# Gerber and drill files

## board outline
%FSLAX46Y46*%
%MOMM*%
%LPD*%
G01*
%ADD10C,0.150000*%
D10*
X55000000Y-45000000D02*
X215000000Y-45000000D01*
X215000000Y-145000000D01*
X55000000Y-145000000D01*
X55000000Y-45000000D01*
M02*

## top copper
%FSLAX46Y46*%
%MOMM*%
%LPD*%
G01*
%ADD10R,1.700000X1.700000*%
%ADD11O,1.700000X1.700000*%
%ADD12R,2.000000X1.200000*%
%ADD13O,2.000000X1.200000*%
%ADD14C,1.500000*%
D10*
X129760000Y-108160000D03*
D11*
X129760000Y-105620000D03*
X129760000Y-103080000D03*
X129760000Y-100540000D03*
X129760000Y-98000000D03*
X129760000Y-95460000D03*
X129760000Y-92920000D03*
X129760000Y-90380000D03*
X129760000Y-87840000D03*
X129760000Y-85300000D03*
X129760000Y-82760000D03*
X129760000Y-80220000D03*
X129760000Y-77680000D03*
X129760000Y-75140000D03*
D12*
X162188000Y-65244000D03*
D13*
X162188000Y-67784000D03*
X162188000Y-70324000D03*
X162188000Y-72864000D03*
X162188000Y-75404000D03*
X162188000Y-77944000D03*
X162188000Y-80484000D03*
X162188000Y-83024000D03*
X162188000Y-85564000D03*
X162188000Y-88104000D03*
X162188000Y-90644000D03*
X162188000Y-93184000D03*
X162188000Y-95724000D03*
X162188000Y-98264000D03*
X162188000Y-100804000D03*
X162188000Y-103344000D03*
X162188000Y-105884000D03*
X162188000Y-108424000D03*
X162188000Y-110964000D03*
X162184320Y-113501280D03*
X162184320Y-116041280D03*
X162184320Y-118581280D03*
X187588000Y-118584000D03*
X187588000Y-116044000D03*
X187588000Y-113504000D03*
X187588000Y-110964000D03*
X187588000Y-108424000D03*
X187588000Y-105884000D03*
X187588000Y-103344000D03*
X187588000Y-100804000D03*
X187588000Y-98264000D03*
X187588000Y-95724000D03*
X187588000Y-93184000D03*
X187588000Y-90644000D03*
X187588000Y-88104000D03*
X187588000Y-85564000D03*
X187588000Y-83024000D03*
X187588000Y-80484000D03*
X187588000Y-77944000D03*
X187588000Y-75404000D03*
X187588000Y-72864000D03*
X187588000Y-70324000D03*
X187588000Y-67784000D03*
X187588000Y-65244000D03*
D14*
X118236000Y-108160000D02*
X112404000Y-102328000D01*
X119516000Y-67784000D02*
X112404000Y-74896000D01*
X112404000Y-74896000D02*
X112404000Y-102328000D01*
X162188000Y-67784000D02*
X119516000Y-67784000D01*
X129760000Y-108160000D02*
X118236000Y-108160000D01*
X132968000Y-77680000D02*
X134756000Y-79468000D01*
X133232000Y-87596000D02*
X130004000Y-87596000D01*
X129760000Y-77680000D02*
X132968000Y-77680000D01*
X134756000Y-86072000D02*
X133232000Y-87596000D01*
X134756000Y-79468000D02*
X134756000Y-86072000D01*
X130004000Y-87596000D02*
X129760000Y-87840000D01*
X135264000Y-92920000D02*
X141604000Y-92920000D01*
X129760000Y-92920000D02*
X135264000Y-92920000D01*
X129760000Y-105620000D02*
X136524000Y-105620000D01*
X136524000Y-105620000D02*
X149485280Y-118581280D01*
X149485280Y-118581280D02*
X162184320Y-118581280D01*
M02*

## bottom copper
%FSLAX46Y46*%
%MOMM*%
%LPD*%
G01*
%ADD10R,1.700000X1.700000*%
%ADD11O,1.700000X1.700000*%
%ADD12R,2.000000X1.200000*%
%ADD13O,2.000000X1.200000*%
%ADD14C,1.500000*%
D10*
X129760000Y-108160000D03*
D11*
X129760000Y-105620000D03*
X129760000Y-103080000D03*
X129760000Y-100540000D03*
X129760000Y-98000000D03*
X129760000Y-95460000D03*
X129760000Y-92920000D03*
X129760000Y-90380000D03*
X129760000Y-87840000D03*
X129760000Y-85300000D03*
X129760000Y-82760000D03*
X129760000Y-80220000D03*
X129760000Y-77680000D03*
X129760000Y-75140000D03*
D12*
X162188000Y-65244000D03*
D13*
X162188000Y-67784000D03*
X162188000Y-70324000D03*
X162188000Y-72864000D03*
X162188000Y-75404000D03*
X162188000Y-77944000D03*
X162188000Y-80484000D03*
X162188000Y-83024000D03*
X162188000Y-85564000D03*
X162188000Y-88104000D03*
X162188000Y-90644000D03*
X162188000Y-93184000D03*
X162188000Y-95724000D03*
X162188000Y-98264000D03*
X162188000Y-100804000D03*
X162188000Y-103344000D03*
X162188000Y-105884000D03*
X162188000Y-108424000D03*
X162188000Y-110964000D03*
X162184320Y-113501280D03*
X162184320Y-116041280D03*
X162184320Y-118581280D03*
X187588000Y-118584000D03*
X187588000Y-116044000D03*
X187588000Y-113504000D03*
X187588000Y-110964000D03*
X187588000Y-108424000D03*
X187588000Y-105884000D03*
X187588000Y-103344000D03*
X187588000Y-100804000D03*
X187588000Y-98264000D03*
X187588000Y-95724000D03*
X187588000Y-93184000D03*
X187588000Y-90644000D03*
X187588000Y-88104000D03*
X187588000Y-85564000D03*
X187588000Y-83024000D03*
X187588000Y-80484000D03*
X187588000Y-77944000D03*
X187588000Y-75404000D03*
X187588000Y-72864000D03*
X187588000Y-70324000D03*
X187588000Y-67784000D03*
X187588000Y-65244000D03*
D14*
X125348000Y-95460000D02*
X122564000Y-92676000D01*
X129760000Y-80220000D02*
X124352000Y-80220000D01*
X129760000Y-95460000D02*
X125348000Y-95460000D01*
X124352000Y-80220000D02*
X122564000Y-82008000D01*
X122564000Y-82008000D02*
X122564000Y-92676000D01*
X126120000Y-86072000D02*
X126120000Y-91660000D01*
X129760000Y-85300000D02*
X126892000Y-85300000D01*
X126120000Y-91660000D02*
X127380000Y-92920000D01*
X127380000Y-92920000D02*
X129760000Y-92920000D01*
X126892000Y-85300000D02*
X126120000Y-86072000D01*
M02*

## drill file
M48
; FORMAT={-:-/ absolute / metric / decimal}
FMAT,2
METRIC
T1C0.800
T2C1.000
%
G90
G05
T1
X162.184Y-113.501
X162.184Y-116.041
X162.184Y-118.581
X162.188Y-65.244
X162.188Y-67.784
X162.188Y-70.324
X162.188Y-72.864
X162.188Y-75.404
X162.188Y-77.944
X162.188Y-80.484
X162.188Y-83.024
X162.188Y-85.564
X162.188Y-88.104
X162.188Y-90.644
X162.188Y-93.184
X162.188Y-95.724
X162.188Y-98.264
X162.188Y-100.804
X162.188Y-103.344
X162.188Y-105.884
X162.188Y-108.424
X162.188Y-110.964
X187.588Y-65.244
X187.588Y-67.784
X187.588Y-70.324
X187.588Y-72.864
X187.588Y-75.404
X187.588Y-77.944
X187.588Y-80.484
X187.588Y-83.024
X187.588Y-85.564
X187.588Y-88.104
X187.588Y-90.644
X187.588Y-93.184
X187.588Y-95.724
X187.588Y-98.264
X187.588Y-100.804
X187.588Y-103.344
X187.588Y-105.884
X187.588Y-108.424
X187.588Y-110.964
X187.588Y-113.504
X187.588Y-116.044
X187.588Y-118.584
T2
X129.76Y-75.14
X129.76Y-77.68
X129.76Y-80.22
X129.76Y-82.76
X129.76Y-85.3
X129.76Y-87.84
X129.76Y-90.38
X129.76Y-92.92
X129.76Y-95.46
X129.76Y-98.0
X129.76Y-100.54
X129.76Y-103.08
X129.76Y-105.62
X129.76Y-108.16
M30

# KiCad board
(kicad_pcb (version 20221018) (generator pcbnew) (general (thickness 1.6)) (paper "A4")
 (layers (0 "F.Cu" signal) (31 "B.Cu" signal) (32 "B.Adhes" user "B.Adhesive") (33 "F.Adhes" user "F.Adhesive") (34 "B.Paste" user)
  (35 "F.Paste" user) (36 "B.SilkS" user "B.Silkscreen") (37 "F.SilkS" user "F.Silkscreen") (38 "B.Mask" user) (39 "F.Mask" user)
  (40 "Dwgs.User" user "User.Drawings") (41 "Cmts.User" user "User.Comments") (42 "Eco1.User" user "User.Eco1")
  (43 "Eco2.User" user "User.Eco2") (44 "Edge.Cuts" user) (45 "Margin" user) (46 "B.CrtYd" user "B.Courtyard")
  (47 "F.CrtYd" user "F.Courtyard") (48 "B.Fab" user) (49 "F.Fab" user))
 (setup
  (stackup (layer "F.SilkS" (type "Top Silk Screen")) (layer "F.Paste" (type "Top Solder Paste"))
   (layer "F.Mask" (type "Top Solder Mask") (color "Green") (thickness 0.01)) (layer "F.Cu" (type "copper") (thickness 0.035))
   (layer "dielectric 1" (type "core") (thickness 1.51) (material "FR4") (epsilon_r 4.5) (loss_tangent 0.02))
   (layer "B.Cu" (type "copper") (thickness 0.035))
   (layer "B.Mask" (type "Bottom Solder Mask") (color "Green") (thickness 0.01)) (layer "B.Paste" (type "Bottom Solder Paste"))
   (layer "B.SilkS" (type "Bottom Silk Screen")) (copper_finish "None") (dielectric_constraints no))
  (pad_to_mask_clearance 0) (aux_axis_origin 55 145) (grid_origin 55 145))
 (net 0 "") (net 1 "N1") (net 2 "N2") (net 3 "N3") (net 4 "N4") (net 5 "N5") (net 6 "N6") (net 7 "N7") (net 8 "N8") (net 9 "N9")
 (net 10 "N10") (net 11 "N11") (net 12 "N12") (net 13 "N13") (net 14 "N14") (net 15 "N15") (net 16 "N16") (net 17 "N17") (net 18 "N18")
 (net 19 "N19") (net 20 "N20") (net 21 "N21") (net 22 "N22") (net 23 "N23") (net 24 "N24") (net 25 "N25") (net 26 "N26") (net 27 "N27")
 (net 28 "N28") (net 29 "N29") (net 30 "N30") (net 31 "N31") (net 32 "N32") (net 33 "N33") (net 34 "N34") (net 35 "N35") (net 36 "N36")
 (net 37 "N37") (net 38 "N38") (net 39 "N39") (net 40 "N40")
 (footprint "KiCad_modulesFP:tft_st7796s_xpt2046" (layer "F.Cu") (at 129.76 108.16 180)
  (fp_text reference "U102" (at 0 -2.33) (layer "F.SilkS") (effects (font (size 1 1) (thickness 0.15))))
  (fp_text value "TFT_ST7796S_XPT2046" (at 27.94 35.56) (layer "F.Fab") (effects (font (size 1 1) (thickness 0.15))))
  (pad "1" thru_hole rect (at 0 0 180) (size 1.7 1.7) (drill 1) (layers "*.Cu" "*.Mask") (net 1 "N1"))
  (pad "2" thru_hole oval (at 0 2.54 180) (size 1.7 1.7) (drill 1) (layers "*.Cu" "*.Mask") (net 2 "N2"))
  (pad "3" thru_hole oval (at 0 5.08 180) (size 1.7 1.7) (drill 1) (layers "*.Cu" "*.Mask") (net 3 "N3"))
  (pad "4" thru_hole oval (at 0 7.62 180) (size 1.7 1.7) (drill 1) (layers "*.Cu" "*.Mask") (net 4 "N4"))
  (pad "5" thru_hole oval (at 0 10.16 180) (size 1.7 1.7) (drill 1) (layers "*.Cu" "*.Mask") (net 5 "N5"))
  (pad "6" thru_hole oval (at 0 12.7 180) (size 1.7 1.7) (drill 1) (layers "*.Cu" "*.Mask") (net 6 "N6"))
  (pad "7" thru_hole oval (at 0 15.24 180) (size 1.7 1.7) (drill 1) (layers "*.Cu" "*.Mask") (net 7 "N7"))
  (pad "8" thru_hole oval (at 0 17.78 180) (size 1.7 1.7) (drill 1) (layers "*.Cu" "*.Mask") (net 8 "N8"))
  (pad "9" thru_hole oval (at 0 20.32 180) (size 1.7 1.7) (drill 1) (layers "*.Cu" "*.Mask") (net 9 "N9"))
  (pad "10" thru_hole oval (at 0 22.86 180) (size 1.7 1.7) (drill 1) (layers "*.Cu" "*.Mask") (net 7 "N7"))
  (pad "11" thru_hole oval (at 0 25.4 180) (size 1.7 1.7) (drill 1) (layers "*.Cu" "*.Mask") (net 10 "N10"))
  (pad "12" thru_hole oval (at 0 27.94 180) (size 1.7 1.7) (drill 1) (layers "*.Cu" "*.Mask") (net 6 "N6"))
  (pad "13" thru_hole oval (at 0 30.48 180) (size 1.7 1.7) (drill 1) (layers "*.Cu" "*.Mask") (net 9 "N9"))
  (pad "14" thru_hole oval (at 0 33.02 180) (size 1.7 1.7) (drill 1) (layers "*.Cu" "*.Mask") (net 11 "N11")))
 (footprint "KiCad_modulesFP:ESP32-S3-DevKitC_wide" (layer "F.Cu") (at 162.188 65.244)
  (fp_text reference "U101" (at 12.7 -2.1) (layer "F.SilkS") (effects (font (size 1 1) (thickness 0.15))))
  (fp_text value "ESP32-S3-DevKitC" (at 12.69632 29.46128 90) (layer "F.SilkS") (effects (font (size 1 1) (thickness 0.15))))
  (pad "1" thru_hole rect (at 0 0 270) (size 1.2 2) (drill 0.8) (layers "*.Cu" "*.Mask") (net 1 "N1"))
  (pad "2" thru_hole oval (at 0 2.54 270) (size 1.2 2) (drill 0.8) (layers "*.Cu" "*.Mask") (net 1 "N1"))
  (pad "3" thru_hole oval (at 0 5.08 270) (size 1.2 2) (drill 0.8) (layers "*.Cu" "*.Mask") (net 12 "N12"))
  (pad "4" thru_hole oval (at 0 7.62 270) (size 1.2 2) (drill 0.8) (layers "*.Cu" "*.Mask") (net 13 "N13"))
  (pad "5" thru_hole oval (at 0 10.16 270) (size 1.2 2) (drill 0.8) (layers "*.Cu" "*.Mask") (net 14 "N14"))
  (pad "6" thru_hole oval (at 0 12.7 270) (size 1.2 2) (drill 0.8) (layers "*.Cu" "*.Mask") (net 10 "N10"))
  (pad "7" thru_hole oval (at 0 15.24 270) (size 1.2 2) (drill 0.8) (layers "*.Cu" "*.Mask") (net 11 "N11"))
  (pad "8" thru_hole oval (at 0 17.78 270) (size 1.2 2) (drill 0.8) (layers "*.Cu" "*.Mask") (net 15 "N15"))
  (pad "9" thru_hole oval (at 0 20.32 270) (size 1.2 2) (drill 0.8) (layers "*.Cu" "*.Mask") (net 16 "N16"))
  (pad "10" thru_hole oval (at 0 22.86 270) (size 1.2 2) (drill 0.8) (layers "*.Cu" "*.Mask") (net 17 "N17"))
  (pad "11" thru_hole oval (at 0 25.4 270) (size 1.2 2) (drill 0.8) (layers "*.Cu" "*.Mask") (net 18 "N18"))
  (pad "12" thru_hole oval (at 0 27.94 270) (size 1.2 2) (drill 0.8) (layers "*.Cu" "*.Mask") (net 9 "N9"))
  (pad "13" thru_hole oval (at 0 30.48 270) (size 1.2 2) (drill 0.8) (layers "*.Cu" "*.Mask") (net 8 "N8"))
  (pad "14" thru_hole oval (at 0 33.02 270) (size 1.2 2) (drill 0.8) (layers "*.Cu" "*.Mask") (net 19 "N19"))
  (pad "15" thru_hole oval (at 0 35.56 270) (size 1.2 2) (drill 0.8) (layers "*.Cu" "*.Mask") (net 5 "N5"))
  (pad "16" thru_hole oval (at 0 38.1 270) (size 1.2 2) (drill 0.8) (layers "*.Cu" "*.Mask") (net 3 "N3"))
  (pad "17" thru_hole oval (at 0 40.64 270) (size 1.2 2) (drill 0.8) (layers "*.Cu" "*.Mask") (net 6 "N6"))
  (pad "18" thru_hole oval (at 0 43.18 270) (size 1.2 2) (drill 0.8) (layers "*.Cu" "*.Mask") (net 7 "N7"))
  (pad "19" thru_hole oval (at 0 45.72 270) (size 1.2 2) (drill 0.8) (layers "*.Cu" "*.Mask") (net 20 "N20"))
  (pad "20" thru_hole oval (at -0.00368 48.25728 270) (size 1.2 2) (drill 0.8) (layers "*.Cu" "*.Mask") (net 4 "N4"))
  (pad "21" thru_hole oval (at -0.00368 50.79728 270) (size 1.2 2) (drill 0.8) (layers "*.Cu" "*.Mask") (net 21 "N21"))
  (pad "22" thru_hole oval (at -0.00368 53.33728 270) (size 1.2 2) (drill 0.8) (layers "*.Cu" "*.Mask") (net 2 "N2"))
  (pad "23" thru_hole oval (at 25.4 53.34 270) (size 1.2 2) (drill 0.8) (layers "*.Cu" "*.Mask") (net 2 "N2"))
  (pad "24" thru_hole oval (at 25.4 50.8 270) (size 1.2 2) (drill 0.8) (layers "*.Cu" "*.Mask") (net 2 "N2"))
  (pad "25" thru_hole oval (at 25.4 48.26 270) (size 1.2 2) (drill 0.8) (layers "*.Cu" "*.Mask") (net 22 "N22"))
  (pad "26" thru_hole oval (at 25.4 45.72 270) (size 1.2 2) (drill 0.8) (layers "*.Cu" "*.Mask") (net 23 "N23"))
  (pad "27" thru_hole oval (at 25.4 43.18 270) (size 1.2 2) (drill 0.8) (layers "*.Cu" "*.Mask") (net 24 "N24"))
  (pad "28" thru_hole oval (at 25.4 40.64 270) (size 1.2 2) (drill 0.8) (layers "*.Cu" "*.Mask") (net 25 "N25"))
  (pad "29" thru_hole oval (at 25.4 38.1 270) (size 1.2 2) (drill 0.8) (layers "*.Cu" "*.Mask") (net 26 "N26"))
  (pad "30" thru_hole oval (at 25.4 35.56 270) (size 1.2 2) (drill 0.8) (layers "*.Cu" "*.Mask") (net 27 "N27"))
  (pad "31" thru_hole oval (at 25.4 33.02 270) (size 1.2 2) (drill 0.8) (layers "*.Cu" "*.Mask") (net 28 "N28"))
  (pad "32" thru_hole oval (at 25.4 30.48 270) (size 1.2 2) (drill 0.8) (layers "*.Cu" "*.Mask") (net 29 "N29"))
  (pad "33" thru_hole oval (at 25.4 27.94 270) (size 1.2 2) (drill 0.8) (layers "*.Cu" "*.Mask") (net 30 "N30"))
  (pad "34" thru_hole oval (at 25.4 25.4 270) (size 1.2 2) (drill 0.8) (layers "*.Cu" "*.Mask") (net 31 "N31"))
  (pad "35" thru_hole oval (at 25.4 22.86 270) (size 1.2 2) (drill 0.8) (layers "*.Cu" "*.Mask") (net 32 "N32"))
  (pad "36" thru_hole oval (at 25.4 20.32 270) (size 1.2 2) (drill 0.8) (layers "*.Cu" "*.Mask") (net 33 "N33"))
  (pad "37" thru_hole oval (at 25.4 17.78 270) (size 1.2 2) (drill 0.8) (layers "*.Cu" "*.Mask") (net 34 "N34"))
  (pad "38" thru_hole oval (at 25.4 15.24 270) (size 1.2 2) (drill 0.8) (layers "*.Cu" "*.Mask") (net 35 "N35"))
  (pad "39" thru_hole oval (at 25.4 12.7 270) (size 1.2 2) (drill 0.8) (layers "*.Cu" "*.Mask") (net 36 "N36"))
  (pad "40" thru_hole oval (at 25.4 10.16 270) (size 1.2 2) (drill 0.8) (layers "*.Cu" "*.Mask") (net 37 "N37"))
  (pad "41" thru_hole oval (at 25.4 7.62 270) (size 1.2 2) (drill 0.8) (layers "*.Cu" "*.Mask") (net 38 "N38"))
  (pad "42" thru_hole oval (at 25.4 5.08 270) (size 1.2 2) (drill 0.8) (layers "*.Cu" "*.Mask") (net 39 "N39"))
  (pad "43" thru_hole oval (at 25.4 2.54 270) (size 1.2 2) (drill 0.8) (layers "*.Cu" "*.Mask") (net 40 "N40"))
  (pad "44" thru_hole oval (at 25.4 0 270) (size 1.2 2) (drill 0.8) (layers "*.Cu" "*.Mask") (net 2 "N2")))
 (gr_rect locked (start 55 45) (end 215 145) (stroke (width 0.15) (type solid)) (fill none) (layer "Edge.Cuts"))
 (segment (start 118.236 108.16) (end 112.404 102.328) (width 1.5) (layer "F.Cu") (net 1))
 (segment (start 119.516 67.784) (end 112.404 74.896) (width 1.5) (layer "F.Cu") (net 1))
 (segment (start 112.404 74.896) (end 112.404 102.328) (width 1.5) (layer "F.Cu") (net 1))
 (segment (start 162.188 67.784) (end 119.516 67.784) (width 1.5) (layer "F.Cu") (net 1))
 (segment (start 129.76 108.16) (end 118.236 108.16) (width 1.5) (layer "F.Cu") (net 1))
 (segment (start 132.968 77.68) (end 134.756 79.468) (width 1.5) (layer "F.Cu") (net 9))
 (segment (start 133.232 87.596) (end 130.004 87.596) (width 1.5) (layer "F.Cu") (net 9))
 (segment (start 129.76 77.68) (end 132.968 77.68) (width 1.5) (layer "F.Cu") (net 9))
 (segment (start 134.756 86.072) (end 133.232 87.596) (width 1.5) (layer "F.Cu") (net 9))
 (segment (start 134.756 79.468) (end 134.756 86.072) (width 1.5) (layer "F.Cu") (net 9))
 (segment (start 130.004 87.596) (end 129.76 87.84) (width 1.5) (layer "F.Cu") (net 9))
 (segment (start 125.348 95.46) (end 122.564 92.676) (width 1.5) (layer "B.Cu") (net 6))
 (segment (start 129.76 80.22) (end 124.352 80.22) (width 1.5) (layer "B.Cu") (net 6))
 (segment (start 129.76 95.46) (end 125.348 95.46) (width 1.5) (layer "B.Cu") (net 6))
 (segment (start 124.352 80.22) (end 122.564 82.008) (width 1.5) (layer "B.Cu") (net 6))
 (segment (start 122.564 82.008) (end 122.564 92.676) (width 1.5) (layer "B.Cu") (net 6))
 (segment (start 135.264 92.92) (end 141.604 92.92) (width 1.5) (layer "F.Cu") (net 7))
 (segment (start 129.76 92.92) (end 135.264 92.92) (width 1.5) (layer "F.Cu") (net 7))
 (segment (start 126.12 86.072) (end 126.12 91.66) (width 1.5) (layer "B.Cu") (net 7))
 (segment (start 129.76 85.3) (end 126.892 85.3) (width 1.5) (layer "B.Cu") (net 7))
 (segment (start 126.12 91.66) (end 127.38 92.92) (width 1.5) (layer "B.Cu") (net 7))
 (segment (start 127.38 92.92) (end 129.76 92.92) (width 1.5) (layer "B.Cu") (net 7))
 (segment (start 126.892 85.3) (end 126.12 86.072) (width 1.5) (layer "B.Cu") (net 7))
 (segment (start 129.76 105.62) (end 136.524 105.62) (width 1.5) (layer "F.Cu") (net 2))
 (segment (start 136.524 105.62) (end 149.48528 118.58128) (width 1.5) (layer "F.Cu") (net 2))
 (segment (start 149.48528 118.58128) (end 162.18432 118.58128) (width 1.5) (layer "F.Cu") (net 2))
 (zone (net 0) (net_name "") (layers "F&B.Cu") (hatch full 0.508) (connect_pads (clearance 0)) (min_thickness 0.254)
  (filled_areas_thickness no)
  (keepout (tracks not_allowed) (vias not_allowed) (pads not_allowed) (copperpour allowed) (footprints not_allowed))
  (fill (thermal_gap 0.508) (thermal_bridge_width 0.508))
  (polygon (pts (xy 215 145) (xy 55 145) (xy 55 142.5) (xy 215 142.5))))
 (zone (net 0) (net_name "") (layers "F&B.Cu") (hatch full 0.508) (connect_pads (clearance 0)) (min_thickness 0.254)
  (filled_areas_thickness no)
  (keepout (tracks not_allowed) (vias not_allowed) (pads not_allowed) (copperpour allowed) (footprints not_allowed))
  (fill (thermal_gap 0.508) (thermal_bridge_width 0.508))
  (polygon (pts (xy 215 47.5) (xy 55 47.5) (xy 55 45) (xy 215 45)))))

